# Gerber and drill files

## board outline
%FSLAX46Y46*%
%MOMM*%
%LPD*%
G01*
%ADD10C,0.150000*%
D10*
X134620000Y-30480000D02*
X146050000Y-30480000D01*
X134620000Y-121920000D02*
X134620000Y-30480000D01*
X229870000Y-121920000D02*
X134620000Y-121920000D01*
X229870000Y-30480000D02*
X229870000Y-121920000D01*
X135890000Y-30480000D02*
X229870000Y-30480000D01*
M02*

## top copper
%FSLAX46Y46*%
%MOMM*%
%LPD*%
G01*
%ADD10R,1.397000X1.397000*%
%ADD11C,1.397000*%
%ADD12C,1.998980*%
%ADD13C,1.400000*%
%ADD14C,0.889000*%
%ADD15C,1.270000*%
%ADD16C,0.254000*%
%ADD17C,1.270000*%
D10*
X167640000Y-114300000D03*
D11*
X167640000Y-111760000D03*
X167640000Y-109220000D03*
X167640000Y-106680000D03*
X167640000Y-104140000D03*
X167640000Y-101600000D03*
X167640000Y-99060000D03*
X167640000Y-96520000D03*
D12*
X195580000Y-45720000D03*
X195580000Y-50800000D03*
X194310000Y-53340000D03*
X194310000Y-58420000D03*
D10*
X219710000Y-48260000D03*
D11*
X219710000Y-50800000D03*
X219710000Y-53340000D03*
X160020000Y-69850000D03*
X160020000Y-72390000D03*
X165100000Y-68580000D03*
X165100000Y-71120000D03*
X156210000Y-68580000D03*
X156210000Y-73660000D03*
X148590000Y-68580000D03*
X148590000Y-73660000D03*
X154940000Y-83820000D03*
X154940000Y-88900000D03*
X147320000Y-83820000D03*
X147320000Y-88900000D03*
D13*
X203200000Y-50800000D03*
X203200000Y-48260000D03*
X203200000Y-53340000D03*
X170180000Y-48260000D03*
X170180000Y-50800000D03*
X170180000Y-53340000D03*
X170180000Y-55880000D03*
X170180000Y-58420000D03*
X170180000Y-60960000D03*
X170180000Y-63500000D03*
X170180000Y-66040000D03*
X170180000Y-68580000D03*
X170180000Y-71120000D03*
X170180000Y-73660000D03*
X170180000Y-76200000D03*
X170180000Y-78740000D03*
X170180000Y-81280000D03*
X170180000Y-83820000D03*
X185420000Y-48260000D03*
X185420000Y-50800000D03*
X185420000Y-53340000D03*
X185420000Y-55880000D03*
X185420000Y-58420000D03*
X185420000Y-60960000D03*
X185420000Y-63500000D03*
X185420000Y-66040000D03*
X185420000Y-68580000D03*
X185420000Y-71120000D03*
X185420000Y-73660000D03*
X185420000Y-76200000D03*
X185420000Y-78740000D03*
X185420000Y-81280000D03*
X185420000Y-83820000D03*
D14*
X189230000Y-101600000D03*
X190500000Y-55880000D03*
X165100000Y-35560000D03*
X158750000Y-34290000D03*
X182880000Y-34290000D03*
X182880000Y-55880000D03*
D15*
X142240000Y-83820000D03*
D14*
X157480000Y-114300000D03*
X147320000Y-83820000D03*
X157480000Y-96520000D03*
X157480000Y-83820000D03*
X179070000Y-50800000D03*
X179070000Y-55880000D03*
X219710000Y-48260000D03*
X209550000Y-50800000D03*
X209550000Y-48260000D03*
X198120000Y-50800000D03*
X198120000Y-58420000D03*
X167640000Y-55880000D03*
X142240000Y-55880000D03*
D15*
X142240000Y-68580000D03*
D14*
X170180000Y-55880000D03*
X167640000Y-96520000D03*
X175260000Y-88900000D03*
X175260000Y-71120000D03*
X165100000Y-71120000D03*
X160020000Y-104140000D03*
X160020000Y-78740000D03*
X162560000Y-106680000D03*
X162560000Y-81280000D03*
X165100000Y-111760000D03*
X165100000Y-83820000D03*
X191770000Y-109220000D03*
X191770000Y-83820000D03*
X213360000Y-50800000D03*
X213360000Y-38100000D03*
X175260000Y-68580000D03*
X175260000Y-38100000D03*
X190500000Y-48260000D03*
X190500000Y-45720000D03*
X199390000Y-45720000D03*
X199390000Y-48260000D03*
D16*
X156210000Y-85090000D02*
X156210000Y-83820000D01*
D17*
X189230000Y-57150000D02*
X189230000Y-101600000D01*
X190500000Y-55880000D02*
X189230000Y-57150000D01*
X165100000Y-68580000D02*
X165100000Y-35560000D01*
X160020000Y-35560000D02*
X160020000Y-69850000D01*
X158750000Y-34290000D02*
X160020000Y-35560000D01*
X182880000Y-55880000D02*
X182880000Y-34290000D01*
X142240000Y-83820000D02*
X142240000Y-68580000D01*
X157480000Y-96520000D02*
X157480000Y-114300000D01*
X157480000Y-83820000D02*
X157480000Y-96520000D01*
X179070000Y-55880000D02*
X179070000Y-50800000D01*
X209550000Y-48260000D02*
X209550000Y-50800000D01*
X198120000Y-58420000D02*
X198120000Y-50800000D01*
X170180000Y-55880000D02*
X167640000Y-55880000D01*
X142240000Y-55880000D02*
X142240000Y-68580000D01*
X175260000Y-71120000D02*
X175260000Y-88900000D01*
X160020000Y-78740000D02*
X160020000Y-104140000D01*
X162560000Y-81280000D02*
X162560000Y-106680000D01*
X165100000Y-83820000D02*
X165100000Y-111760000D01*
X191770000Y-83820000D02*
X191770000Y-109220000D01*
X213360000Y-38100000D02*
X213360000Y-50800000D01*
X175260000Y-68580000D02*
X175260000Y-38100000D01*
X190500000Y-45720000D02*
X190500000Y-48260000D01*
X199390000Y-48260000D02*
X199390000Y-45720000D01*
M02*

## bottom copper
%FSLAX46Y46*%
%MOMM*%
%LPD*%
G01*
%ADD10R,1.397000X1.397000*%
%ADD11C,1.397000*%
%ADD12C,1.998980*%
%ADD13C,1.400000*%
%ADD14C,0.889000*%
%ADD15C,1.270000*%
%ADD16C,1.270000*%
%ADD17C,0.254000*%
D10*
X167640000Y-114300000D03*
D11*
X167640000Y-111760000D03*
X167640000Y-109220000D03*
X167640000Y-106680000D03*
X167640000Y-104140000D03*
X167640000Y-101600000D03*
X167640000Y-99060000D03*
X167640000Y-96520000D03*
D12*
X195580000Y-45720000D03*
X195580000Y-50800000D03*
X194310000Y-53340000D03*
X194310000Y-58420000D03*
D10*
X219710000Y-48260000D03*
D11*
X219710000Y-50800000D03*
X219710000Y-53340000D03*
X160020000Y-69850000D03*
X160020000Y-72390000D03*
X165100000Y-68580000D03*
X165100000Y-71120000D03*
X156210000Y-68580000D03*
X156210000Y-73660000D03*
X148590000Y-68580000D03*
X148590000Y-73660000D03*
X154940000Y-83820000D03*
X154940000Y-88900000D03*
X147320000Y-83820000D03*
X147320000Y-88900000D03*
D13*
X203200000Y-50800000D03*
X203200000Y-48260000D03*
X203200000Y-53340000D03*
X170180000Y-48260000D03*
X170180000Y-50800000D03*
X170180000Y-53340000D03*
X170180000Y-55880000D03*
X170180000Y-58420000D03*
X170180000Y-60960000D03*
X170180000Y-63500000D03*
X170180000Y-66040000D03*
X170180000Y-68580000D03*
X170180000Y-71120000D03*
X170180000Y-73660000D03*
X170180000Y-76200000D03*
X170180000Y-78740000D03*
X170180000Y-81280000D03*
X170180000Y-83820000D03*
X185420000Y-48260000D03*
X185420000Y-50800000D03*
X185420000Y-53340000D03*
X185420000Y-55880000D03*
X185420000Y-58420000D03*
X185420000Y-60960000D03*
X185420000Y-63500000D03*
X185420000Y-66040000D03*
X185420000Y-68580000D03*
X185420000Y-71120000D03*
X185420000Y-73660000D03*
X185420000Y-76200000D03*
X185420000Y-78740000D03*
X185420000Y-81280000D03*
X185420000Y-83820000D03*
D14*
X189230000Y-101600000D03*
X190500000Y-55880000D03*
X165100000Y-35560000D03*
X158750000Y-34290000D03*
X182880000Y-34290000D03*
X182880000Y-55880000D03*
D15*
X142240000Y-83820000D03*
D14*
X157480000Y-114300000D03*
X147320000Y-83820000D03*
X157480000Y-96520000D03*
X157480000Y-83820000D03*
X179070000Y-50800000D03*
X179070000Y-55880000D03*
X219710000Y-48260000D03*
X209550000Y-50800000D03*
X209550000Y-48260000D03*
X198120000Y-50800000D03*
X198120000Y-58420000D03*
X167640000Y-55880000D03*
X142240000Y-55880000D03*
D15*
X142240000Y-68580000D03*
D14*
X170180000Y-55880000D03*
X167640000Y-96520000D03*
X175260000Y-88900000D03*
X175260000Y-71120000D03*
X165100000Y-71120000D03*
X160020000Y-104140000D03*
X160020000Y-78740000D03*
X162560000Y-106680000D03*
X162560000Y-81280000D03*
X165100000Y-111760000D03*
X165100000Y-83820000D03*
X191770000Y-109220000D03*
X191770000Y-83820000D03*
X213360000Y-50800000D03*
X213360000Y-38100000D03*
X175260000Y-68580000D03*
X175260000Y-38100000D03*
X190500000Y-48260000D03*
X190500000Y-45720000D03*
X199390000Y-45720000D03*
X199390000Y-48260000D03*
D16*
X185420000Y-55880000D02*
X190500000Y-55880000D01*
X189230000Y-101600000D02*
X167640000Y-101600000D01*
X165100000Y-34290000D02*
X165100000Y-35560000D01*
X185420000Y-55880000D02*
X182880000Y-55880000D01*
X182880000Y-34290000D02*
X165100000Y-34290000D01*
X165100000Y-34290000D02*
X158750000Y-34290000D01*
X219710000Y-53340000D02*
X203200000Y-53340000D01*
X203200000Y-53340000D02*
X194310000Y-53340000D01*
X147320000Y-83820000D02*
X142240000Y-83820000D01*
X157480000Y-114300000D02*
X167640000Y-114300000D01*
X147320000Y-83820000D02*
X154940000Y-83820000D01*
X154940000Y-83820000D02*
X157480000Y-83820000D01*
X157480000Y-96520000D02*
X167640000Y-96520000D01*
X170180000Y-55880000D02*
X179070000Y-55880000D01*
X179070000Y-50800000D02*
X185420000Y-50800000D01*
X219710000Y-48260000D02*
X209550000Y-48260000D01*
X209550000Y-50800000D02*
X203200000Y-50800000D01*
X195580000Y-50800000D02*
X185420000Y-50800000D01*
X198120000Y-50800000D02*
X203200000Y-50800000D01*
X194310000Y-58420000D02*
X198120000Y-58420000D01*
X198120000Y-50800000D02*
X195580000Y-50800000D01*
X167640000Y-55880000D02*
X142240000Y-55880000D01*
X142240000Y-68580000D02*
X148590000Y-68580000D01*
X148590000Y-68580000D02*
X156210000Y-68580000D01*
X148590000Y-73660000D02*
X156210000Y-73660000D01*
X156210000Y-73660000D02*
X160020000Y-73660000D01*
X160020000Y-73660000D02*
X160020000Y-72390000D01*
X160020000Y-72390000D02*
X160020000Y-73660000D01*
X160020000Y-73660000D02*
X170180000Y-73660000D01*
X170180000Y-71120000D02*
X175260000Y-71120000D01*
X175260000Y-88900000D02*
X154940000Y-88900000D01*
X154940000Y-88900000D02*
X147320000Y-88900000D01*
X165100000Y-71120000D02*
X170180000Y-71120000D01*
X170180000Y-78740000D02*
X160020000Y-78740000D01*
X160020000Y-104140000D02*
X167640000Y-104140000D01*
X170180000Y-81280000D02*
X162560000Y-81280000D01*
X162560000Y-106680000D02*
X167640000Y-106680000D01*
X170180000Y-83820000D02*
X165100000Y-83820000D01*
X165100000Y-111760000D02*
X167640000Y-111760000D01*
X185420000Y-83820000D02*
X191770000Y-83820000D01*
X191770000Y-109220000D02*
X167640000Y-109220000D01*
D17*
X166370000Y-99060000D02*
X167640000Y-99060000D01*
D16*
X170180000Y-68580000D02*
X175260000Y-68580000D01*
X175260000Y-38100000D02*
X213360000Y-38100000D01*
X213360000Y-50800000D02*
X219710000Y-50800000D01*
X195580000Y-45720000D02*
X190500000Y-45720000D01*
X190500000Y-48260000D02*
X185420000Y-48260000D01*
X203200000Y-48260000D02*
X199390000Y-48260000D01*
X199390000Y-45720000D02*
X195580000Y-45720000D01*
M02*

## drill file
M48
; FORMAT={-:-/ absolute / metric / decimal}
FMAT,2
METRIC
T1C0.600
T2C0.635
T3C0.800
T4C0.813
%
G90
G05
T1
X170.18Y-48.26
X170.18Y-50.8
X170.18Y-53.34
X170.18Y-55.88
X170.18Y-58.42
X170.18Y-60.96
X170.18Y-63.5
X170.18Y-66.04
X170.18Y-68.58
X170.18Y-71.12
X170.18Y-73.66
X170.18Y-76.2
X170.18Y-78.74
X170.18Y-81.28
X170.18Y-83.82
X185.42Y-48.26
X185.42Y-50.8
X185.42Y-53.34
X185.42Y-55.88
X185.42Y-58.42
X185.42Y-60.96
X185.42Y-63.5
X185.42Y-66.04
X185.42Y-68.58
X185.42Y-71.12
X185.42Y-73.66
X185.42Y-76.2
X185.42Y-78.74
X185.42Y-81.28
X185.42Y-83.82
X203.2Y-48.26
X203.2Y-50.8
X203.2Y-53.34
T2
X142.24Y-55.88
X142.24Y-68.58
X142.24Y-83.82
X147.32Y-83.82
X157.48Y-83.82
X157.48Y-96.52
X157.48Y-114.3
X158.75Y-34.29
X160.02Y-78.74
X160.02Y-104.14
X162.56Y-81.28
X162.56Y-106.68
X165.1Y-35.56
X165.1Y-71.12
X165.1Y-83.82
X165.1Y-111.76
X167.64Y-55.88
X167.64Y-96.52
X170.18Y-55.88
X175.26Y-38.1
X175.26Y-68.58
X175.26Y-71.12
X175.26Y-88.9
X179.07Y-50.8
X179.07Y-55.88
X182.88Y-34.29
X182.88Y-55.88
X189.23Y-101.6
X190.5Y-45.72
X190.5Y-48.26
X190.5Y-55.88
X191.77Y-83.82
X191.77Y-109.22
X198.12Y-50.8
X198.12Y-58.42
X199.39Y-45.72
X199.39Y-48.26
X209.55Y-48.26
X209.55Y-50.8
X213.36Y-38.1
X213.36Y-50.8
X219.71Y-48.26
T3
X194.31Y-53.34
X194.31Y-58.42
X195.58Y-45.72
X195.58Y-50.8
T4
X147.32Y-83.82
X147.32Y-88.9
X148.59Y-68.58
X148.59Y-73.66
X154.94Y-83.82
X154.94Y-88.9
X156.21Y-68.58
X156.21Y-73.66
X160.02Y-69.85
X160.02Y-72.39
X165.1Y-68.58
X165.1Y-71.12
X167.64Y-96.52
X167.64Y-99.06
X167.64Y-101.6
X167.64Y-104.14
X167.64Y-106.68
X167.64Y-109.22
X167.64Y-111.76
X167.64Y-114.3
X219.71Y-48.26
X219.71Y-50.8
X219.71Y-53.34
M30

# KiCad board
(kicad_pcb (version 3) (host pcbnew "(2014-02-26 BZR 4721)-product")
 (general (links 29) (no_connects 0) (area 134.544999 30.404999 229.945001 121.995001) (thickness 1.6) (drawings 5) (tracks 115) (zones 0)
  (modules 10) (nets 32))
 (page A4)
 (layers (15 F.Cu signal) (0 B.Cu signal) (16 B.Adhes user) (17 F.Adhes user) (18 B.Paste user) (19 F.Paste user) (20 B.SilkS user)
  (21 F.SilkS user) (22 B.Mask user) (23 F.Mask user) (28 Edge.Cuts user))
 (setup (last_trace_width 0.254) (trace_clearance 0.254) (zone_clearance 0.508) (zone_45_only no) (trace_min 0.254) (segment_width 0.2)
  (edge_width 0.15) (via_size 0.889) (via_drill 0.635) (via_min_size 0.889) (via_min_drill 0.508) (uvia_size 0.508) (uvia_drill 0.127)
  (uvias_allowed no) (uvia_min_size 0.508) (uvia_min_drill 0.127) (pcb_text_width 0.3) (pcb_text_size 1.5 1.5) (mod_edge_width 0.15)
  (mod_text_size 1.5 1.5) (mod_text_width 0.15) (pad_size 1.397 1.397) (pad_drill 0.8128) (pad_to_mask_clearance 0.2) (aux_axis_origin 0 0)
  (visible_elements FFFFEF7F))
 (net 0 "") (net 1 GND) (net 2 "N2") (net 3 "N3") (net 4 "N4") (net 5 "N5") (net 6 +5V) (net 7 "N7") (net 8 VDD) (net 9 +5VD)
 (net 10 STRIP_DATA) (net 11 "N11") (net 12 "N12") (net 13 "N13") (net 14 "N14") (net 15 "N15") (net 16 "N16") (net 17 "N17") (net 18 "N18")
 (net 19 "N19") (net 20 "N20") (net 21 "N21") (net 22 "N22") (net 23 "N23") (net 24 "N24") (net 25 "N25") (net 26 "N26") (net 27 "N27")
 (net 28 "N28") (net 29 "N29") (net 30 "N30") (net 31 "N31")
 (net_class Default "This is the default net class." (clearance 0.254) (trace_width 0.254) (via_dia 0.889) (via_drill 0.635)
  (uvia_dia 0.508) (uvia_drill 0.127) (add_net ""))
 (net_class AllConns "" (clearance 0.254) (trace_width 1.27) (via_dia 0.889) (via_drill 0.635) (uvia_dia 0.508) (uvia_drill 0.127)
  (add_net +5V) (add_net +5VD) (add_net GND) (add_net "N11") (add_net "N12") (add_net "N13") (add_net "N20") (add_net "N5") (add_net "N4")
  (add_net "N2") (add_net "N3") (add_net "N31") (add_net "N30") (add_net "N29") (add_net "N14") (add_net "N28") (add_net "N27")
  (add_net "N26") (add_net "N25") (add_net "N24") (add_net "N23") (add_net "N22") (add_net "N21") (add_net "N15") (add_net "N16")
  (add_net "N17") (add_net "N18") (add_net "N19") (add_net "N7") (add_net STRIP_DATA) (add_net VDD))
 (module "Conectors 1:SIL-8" (layer F.Cu) (at 167.64 105.41 90)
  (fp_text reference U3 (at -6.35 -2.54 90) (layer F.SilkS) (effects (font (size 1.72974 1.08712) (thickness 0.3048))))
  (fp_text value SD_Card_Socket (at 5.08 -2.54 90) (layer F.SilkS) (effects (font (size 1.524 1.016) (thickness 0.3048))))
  (pad 8 thru_hole rect (at -8.89 0 90) (size 1.397 1.397) (drill 0.8128) (layers *.Cu *.Mask F.SilkS) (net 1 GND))
  (pad 7 thru_hole circle (at -6.35 0 90) (size 1.397 1.397) (drill 0.8128) (layers *.Cu *.Mask F.SilkS) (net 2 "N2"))
  (pad 6 thru_hole circle (at -3.81 0 90) (size 1.397 1.397) (drill 0.8128) (layers *.Cu *.Mask F.SilkS) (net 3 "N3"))
  (pad 5 thru_hole circle (at -1.27 0 90) (size 1.397 1.397) (drill 0.8128) (layers *.Cu *.Mask F.SilkS) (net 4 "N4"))
  (pad 4 thru_hole circle (at 1.27 0 90) (size 1.397 1.397) (drill 0.8128) (layers *.Cu *.Mask F.SilkS) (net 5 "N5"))
  (pad 3 thru_hole circle (at 3.81 0 90) (size 1.397 1.397) (drill 0.8128) (layers *.Cu *.Mask F.SilkS) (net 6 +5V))
  (pad 2 thru_hole circle (at 6.35 0 90) (size 1.397 1.397) (drill 0.8128) (layers *.Cu *.Mask F.SilkS) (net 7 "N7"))
  (pad 1 thru_hole circle (at 8.89 0 90) (size 1.397 1.397) (drill 0.8128) (layers *.Cu *.Mask F.SilkS) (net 1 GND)))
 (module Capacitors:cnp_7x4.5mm (layer F.Cu) (at 195.58 48.26 270)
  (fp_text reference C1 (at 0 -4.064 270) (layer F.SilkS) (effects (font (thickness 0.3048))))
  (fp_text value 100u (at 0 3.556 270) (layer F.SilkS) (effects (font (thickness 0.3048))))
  (pad 1 thru_hole circle (at -2.54 0 270) (size 1.99898 1.99898) (drill 0.8001) (layers *.Cu *.Mask F.SilkS) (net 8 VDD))
  (pad 2 thru_hole circle (at 2.54 0 270) (size 1.99898 1.99898) (drill 0.8001) (layers *.Cu *.Mask F.SilkS) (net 1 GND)))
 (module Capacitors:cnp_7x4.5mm (layer F.Cu) (at 194.31 55.88 270)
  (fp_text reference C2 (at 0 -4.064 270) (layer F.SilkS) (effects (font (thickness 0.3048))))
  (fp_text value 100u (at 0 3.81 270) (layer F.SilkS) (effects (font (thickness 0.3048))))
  (pad 1 thru_hole circle (at -2.54 0 270) (size 1.99898 1.99898) (drill 0.8001) (layers *.Cu *.Mask F.SilkS) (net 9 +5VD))
  (pad 2 thru_hole circle (at 2.54 0 270) (size 1.99898 1.99898) (drill 0.8001) (layers *.Cu *.Mask F.SilkS) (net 1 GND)))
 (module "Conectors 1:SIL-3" (layer F.Cu) (at 219.71 50.8 270)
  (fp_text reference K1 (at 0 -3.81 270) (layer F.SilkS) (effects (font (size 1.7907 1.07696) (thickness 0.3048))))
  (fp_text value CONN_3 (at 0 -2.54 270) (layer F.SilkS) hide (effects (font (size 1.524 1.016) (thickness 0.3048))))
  (pad 1 thru_hole rect (at -2.54 0 270) (size 1.397 1.397) (drill 0.8128) (layers *.Cu *.Mask F.SilkS) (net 1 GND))
  (pad 2 thru_hole circle (at 0 0 270) (size 1.397 1.397) (drill 0.8128) (layers *.Cu *.Mask F.SilkS) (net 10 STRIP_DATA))
  (pad 3 thru_hole circle (at 2.54 0 270) (size 1.397 1.397) (drill 0.8128) (layers *.Cu *.Mask F.SilkS) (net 9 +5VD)))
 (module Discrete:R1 (layer F.Cu) (at 160.02 71.12 270) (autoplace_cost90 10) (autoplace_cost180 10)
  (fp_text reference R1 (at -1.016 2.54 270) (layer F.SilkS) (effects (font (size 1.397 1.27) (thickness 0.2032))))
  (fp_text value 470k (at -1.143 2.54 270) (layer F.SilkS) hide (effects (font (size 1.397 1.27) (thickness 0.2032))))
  (pad 1 thru_hole circle (at -1.27 0 270) (size 1.397 1.397) (drill 0.8128) (layers *.Cu *.Mask F.SilkS) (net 6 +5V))
  (pad 2 thru_hole circle (at 1.27 0 270) (size 1.397 1.397) (drill 0.8128) (layers *.Cu *.Mask F.SilkS) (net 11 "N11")))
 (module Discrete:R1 (layer F.Cu) (at 165.1 69.85 270) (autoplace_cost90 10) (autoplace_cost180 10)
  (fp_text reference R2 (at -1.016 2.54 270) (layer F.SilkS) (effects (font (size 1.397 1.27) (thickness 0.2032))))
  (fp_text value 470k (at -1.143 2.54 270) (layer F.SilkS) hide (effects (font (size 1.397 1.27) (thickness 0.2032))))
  (pad 1 thru_hole circle (at -1.27 0 270) (size 1.397 1.397) (drill 0.8128) (layers *.Cu *.Mask F.SilkS) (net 6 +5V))
  (pad 2 thru_hole circle (at 1.27 0 270) (size 1.397 1.397) (drill 0.8128) (layers *.Cu *.Mask F.SilkS) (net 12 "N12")))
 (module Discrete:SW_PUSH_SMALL (layer F.Cu) (at 152.4 71.12)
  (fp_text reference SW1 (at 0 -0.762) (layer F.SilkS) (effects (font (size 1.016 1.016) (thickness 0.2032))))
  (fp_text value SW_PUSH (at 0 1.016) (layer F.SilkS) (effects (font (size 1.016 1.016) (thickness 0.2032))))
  (pad 1 thru_hole circle (at 3.81 -2.54) (size 1.397 1.397) (drill 0.8128) (layers *.Cu *.Mask F.SilkS) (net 1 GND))
  (pad 2 thru_hole circle (at 3.81 2.54) (size 1.397 1.397) (drill 0.8128) (layers *.Cu *.Mask F.SilkS) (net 11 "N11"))
  (pad 1 thru_hole circle (at -3.81 -2.54) (size 1.397 1.397) (drill 0.8128) (layers *.Cu *.Mask F.SilkS) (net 1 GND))
  (pad 2 thru_hole circle (at -3.81 2.54) (size 1.397 1.397) (drill 0.8128) (layers *.Cu *.Mask F.SilkS) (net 11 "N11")))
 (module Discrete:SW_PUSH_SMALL (layer F.Cu) (at 151.13 86.36)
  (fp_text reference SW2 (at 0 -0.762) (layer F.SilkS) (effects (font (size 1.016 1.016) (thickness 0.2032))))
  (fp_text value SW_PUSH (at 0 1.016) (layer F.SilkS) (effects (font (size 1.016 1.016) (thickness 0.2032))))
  (pad 1 thru_hole circle (at 3.81 -2.54) (size 1.397 1.397) (drill 0.8128) (layers *.Cu *.Mask F.SilkS) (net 1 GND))
  (pad 2 thru_hole circle (at 3.81 2.54) (size 1.397 1.397) (drill 0.8128) (layers *.Cu *.Mask F.SilkS) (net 12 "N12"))
  (pad 1 thru_hole circle (at -3.81 -2.54) (size 1.397 1.397) (drill 0.8128) (layers *.Cu *.Mask F.SilkS) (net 1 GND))
  (pad 2 thru_hole circle (at -3.81 2.54) (size 1.397 1.397) (drill 0.8128) (layers *.Cu *.Mask F.SilkS) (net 12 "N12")))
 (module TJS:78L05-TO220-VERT (layer F.Cu) (at 208.28 50.8 270)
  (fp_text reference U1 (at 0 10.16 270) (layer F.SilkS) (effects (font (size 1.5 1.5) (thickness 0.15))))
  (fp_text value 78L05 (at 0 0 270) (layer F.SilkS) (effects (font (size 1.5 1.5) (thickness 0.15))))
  (pad 1 thru_hole circle (at 0 5.08 270) (size 1.4 1.4) (drill 0.6) (layers *.Cu *.Mask F.SilkS) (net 1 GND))
  (pad 2 thru_hole circle (at -2.54 5.08 270) (size 1.4 1.4) (drill 0.6) (layers *.Cu *.Mask F.SilkS) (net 8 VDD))
  (pad 3 thru_hole circle (at 2.54 5.08 270) (size 1.4 1.4) (drill 0.6) (layers *.Cu *.Mask F.SilkS) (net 9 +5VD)))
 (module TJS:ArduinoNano (layer F.Cu) (at 177.8 45.72)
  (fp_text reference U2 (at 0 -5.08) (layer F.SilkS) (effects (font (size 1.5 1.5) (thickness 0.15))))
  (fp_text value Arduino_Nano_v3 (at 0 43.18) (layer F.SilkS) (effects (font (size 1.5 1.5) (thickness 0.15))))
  (pad 1 thru_hole circle (at -7.62 2.54) (size 1.4 1.4) (drill 0.6) (layers *.Cu *.Mask F.SilkS) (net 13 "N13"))
  (pad 2 thru_hole circle (at -7.62 5.08) (size 1.4 1.4) (drill 0.6) (layers *.Cu *.Mask F.SilkS) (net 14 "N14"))
  (pad 3 thru_hole circle (at -7.62 7.62) (size 1.4 1.4) (drill 0.6) (layers *.Cu *.Mask F.SilkS) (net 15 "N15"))
  (pad 4 thru_hole circle (at -7.62 10.16) (size 1.4 1.4) (drill 0.6) (layers *.Cu *.Mask F.SilkS) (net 1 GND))
  (pad 5 thru_hole circle (at -7.62 12.7) (size 1.4 1.4) (drill 0.6) (layers *.Cu *.Mask F.SilkS) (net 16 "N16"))
  (pad 6 thru_hole circle (at -7.62 15.24) (size 1.4 1.4) (drill 0.6) (layers *.Cu *.Mask F.SilkS) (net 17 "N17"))
  (pad 7 thru_hole circle (at -7.62 17.78) (size 1.4 1.4) (drill 0.6) (layers *.Cu *.Mask F.SilkS) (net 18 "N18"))
  (pad 8 thru_hole circle (at -7.62 20.32) (size 1.4 1.4) (drill 0.6) (layers *.Cu *.Mask F.SilkS) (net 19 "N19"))
  (pad 9 thru_hole circle (at -7.62 22.86) (size 1.4 1.4) (drill 0.6) (layers *.Cu *.Mask F.SilkS) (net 10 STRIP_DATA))
  (pad 10 thru_hole circle (at -7.62 25.4) (size 1.4 1.4) (drill 0.6) (layers *.Cu *.Mask F.SilkS) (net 12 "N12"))
  (pad 11 thru_hole circle (at -7.62 27.94) (size 1.4 1.4) (drill 0.6) (layers *.Cu *.Mask F.SilkS) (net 11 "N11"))
  (pad 12 thru_hole circle (at -7.62 30.48) (size 1.4 1.4) (drill 0.6) (layers *.Cu *.Mask F.SilkS) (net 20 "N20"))
  (pad 13 thru_hole circle (at -7.62 33.02) (size 1.4 1.4) (drill 0.6) (layers *.Cu *.Mask F.SilkS) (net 5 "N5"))
  (pad 14 thru_hole circle (at -7.62 35.56) (size 1.4 1.4) (drill 0.6) (layers *.Cu *.Mask F.SilkS) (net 4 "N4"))
  (pad 15 thru_hole circle (at -7.62 38.1) (size 1.4 1.4) (drill 0.6) (layers *.Cu *.Mask F.SilkS) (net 2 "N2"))
  (pad 30 thru_hole circle (at 7.62 2.54) (size 1.4 1.4) (drill 0.6) (layers *.Cu *.Mask F.SilkS) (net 8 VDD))
  (pad 29 thru_hole circle (at 7.62 5.08) (size 1.4 1.4) (drill 0.6) (layers *.Cu *.Mask F.SilkS) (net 1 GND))
  (pad 28 thru_hole circle (at 7.62 7.62) (size 1.4 1.4) (drill 0.6) (layers *.Cu *.Mask F.SilkS) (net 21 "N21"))
  (pad 27 thru_hole circle (at 7.62 10.16) (size 1.4 1.4) (drill 0.6) (layers *.Cu *.Mask F.SilkS) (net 6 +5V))
  (pad 26 thru_hole circle (at 7.62 12.7) (size 1.4 1.4) (drill 0.6) (layers *.Cu *.Mask F.SilkS) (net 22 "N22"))
  (pad 25 thru_hole circle (at 7.62 15.24) (size 1.4 1.4) (drill 0.6) (layers *.Cu *.Mask F.SilkS) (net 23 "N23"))
  (pad 24 thru_hole circle (at 7.62 17.78) (size 1.4 1.4) (drill 0.6) (layers *.Cu *.Mask F.SilkS) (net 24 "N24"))
  (pad 23 thru_hole circle (at 7.62 20.32) (size 1.4 1.4) (drill 0.6) (layers *.Cu *.Mask F.SilkS) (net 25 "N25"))
  (pad 22 thru_hole circle (at 7.62 22.86) (size 1.4 1.4) (drill 0.6) (layers *.Cu *.Mask F.SilkS) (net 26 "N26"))
  (pad 21 thru_hole circle (at 7.62 25.4) (size 1.4 1.4) (drill 0.6) (layers *.Cu *.Mask F.SilkS) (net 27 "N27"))
  (pad 20 thru_hole circle (at 7.62 27.94) (size 1.4 1.4) (drill 0.6) (layers *.Cu *.Mask F.SilkS) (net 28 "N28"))
  (pad 19 thru_hole circle (at 7.62 30.48) (size 1.4 1.4) (drill 0.6) (layers *.Cu *.Mask F.SilkS) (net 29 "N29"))
  (pad 18 thru_hole circle (at 7.62 33.02) (size 1.4 1.4) (drill 0.6) (layers *.Cu *.Mask F.SilkS) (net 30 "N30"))
  (pad 17 thru_hole circle (at 7.62 35.56) (size 1.4 1.4) (drill 0.6) (layers *.Cu *.Mask F.SilkS) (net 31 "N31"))
  (pad 16 thru_hole circle (at 7.62 38.1) (size 1.4 1.4) (drill 0.6) (layers *.Cu *.Mask F.SilkS) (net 3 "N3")))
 (gr_line (start 134.62 30.48) (end 146.05 30.48) (angle 90) (layer Edge.Cuts) (width 0.15))
 (gr_line (start 134.62 121.92) (end 134.62 30.48) (angle 90) (layer Edge.Cuts) (width 0.15))
 (gr_line (start 229.87 121.92) (end 134.62 121.92) (angle 90) (layer Edge.Cuts) (width 0.15))
 (gr_line (start 229.87 30.48) (end 229.87 121.92) (angle 90) (layer Edge.Cuts) (width 0.15))
 (gr_line (start 135.89 30.48) (end 229.87 30.48) (angle 90) (layer Edge.Cuts) (width 0.15))
 (segment (start 156.21 85.09) (end 156.21 83.82) (width 0.254) (layer F.Cu) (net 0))
 (segment (start 185.42 55.88) (end 190.5 55.88) (width 1.27) (layer B.Cu) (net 6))
 (segment (start 189.23 101.6) (end 167.64 101.6) (width 1.27) (layer B.Cu) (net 6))
 (via (at 189.23 101.6) (size 0.889) (layers F.Cu B.Cu) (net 6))
 (segment (start 189.23 57.15) (end 189.23 101.6) (width 1.27) (layer F.Cu) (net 6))
 (segment (start 190.5 55.88) (end 189.23 57.15) (width 1.27) (layer F.Cu) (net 6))
 (via (at 190.5 55.88) (size 0.889) (layers F.Cu B.Cu) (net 6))
 (segment (start 165.1 34.29) (end 165.1 35.56) (width 1.27) (layer B.Cu) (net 6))
 (via (at 165.1 35.56) (size 0.889) (layers F.Cu B.Cu) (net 6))
 (segment (start 165.1 68.58) (end 165.1 35.56) (width 1.27) (layer F.Cu) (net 6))
 (segment (start 185.42 55.88) (end 182.88 55.88) (width 1.27) (layer B.Cu) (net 6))
 (segment (start 160.02 35.56) (end 160.02 69.85) (width 1.27) (layer F.Cu) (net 6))
 (segment (start 158.75 34.29) (end 160.02 35.56) (width 1.27) (layer F.Cu) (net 6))
 (via (at 158.75 34.29) (size 0.889) (layers F.Cu B.Cu) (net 6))
 (segment (start 182.88 34.29) (end 165.1 34.29) (width 1.27) (layer B.Cu) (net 6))
 (segment (start 165.1 34.29) (end 158.75 34.29) (width 1.27) (layer B.Cu) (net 6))
 (via (at 182.88 34.29) (size 0.889) (layers F.Cu B.Cu) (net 6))
 (segment (start 182.88 55.88) (end 182.88 34.29) (width 1.27) (layer F.Cu) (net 6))
 (via (at 182.88 55.88) (size 0.889) (layers F.Cu B.Cu) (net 6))
 (segment (start 219.71 53.34) (end 203.2 53.34) (width 1.27) (layer B.Cu) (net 9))
 (segment (start 203.2 53.34) (end 194.31 53.34) (width 1.27) (layer B.Cu) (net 9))
 (segment (start 147.32 83.82) (end 142.24 83.82) (width 1.27) (layer B.Cu) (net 1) (status 400000))
 (via (at 142.24 83.82) (size 1.27) (layers F.Cu B.Cu) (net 1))
 (segment (start 142.24 83.82) (end 142.24 68.58) (width 1.27) (layer F.Cu) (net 1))
 (segment (start 157.48 96.52) (end 157.48 114.3) (width 1.27) (layer F.Cu) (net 1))
 (segment (start 157.48 114.3) (end 167.64 114.3) (width 1.27) (layer B.Cu) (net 1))
 (via (at 157.48 114.3) (size 0.889) (layers F.Cu B.Cu) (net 1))
 (via (at 147.32 83.82) (size 0.889) (layers F.Cu B.Cu) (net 1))
 (segment (start 147.32 83.82) (end 154.94 83.82) (width 1.27) (layer B.Cu) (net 1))
 (segment (start 154.94 83.82) (end 157.48 83.82) (width 1.27) (layer B.Cu) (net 1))
 (segment (start 157.48 96.52) (end 167.64 96.52) (width 1.27) (layer B.Cu) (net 1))
 (via (at 157.48 96.52) (size 0.889) (layers F.Cu B.Cu) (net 1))
 (segment (start 157.48 83.82) (end 157.48 96.52) (width 1.27) (layer F.Cu) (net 1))
 (via (at 157.48 83.82) (size 0.889) (layers F.Cu B.Cu) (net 1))
 (segment (start 170.18 55.88) (end 179.07 55.88) (width 1.27) (layer B.Cu) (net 1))
 (segment (start 179.07 50.8) (end 185.42 50.8) (width 1.27) (layer B.Cu) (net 1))
 (via (at 179.07 50.8) (size 0.889) (layers F.Cu B.Cu) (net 1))
 (segment (start 179.07 55.88) (end 179.07 50.8) (width 1.27) (layer F.Cu) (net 1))
 (via (at 179.07 55.88) (size 0.889) (layers F.Cu B.Cu) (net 1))
 (via (at 219.71 48.26) (size 0.889) (layers F.Cu B.Cu) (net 1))
 (segment (start 219.71 48.26) (end 209.55 48.26) (width 1.27) (layer B.Cu) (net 1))
 (segment (start 209.55 50.8) (end 203.2 50.8) (width 1.27) (layer B.Cu) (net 1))
 (via (at 209.55 50.8) (size 0.889) (layers F.Cu B.Cu) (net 1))
 (segment (start 209.55 48.26) (end 209.55 50.8) (width 1.27) (layer F.Cu) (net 1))
 (via (at 209.55 48.26) (size 0.889) (layers F.Cu B.Cu) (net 1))
 (segment (start 195.58 50.8) (end 185.42 50.8) (width 1.27) (layer B.Cu) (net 1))
 (segment (start 198.12 50.8) (end 203.2 50.8) (width 1.27) (layer B.Cu) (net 1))
 (segment (start 194.31 58.42) (end 198.12 58.42) (width 1.27) (layer B.Cu) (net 1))
 (segment (start 198.12 50.8) (end 195.58 50.8) (width 1.27) (layer B.Cu) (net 1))
 (via (at 198.12 50.8) (size 0.889) (layers F.Cu B.Cu) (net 1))
 (segment (start 198.12 58.42) (end 198.12 50.8) (width 1.27) (layer F.Cu) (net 1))
 (via (at 198.12 58.42) (size 0.889) (layers F.Cu B.Cu) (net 1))
 (segment (start 170.18 55.88) (end 167.64 55.88) (width 1.27) (layer F.Cu) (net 1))
 (via (at 167.64 55.88) (size 0.889) (layers F.Cu B.Cu) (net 1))
 (segment (start 167.64 55.88) (end 142.24 55.88) (width 1.27) (layer B.Cu) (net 1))
 (via (at 142.24 55.88) (size 0.889) (layers F.Cu B.Cu) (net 1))
 (segment (start 142.24 55.88) (end 142.24 68.58) (width 1.27) (layer F.Cu) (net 1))
 (segment (start 142.24 68.58) (end 148.59 68.58) (width 1.27) (layer B.Cu) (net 1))
 (via (at 142.24 68.58) (size 1.27) (layers F.Cu B.Cu) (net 1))
 (segment (start 148.59 68.58) (end 156.21 68.58) (width 1.27) (layer B.Cu) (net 1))
 (via (at 170.18 55.88) (size 0.889) (layers F.Cu B.Cu) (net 1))
 (via (at 167.64 96.52) (size 0.889) (layers F.Cu B.Cu) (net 1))
 (segment (start 148.59 73.66) (end 156.21 73.66) (width 1.27) (layer B.Cu) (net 11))
 (segment (start 156.21 73.66) (end 160.02 73.66) (width 1.27) (layer B.Cu) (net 11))
 (segment (start 160.02 73.66) (end 160.02 72.39) (width 1.27) (layer B.Cu) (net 11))
 (segment (start 160.02 72.39) (end 160.02 73.66) (width 1.27) (layer B.Cu) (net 11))
 (segment (start 160.02 73.66) (end 170.18 73.66) (width 1.27) (layer B.Cu) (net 11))
 (segment (start 170.18 71.12) (end 175.26 71.12) (width 1.27) (layer B.Cu) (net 12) (status 400000))
 (segment (start 175.26 88.9) (end 154.94 88.9) (width 1.27) (layer B.Cu) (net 12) (status 800000))
 (via (at 175.26 88.9) (size 0.889) (layers F.Cu B.Cu) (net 12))
 (segment (start 175.26 71.12) (end 175.26 88.9) (width 1.27) (layer F.Cu) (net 12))
 (via (at 175.26 71.12) (size 0.889) (layers F.Cu B.Cu) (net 12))
 (segment (start 154.94 88.9) (end 147.32 88.9) (width 1.27) (layer B.Cu) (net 12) (status C00000))
 (via (at 165.1 71.12) (size 0.889) (layers F.Cu B.Cu) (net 12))
 (segment (start 165.1 71.12) (end 170.18 71.12) (width 1.27) (layer B.Cu) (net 12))
 (segment (start 170.18 78.74) (end 160.02 78.74) (width 1.27) (layer B.Cu) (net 5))
 (segment (start 160.02 104.14) (end 167.64 104.14) (width 1.27) (layer B.Cu) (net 5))
 (via (at 160.02 104.14) (size 0.889) (layers F.Cu B.Cu) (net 5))
 (segment (start 160.02 78.74) (end 160.02 104.14) (width 1.27) (layer F.Cu) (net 5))
 (via (at 160.02 78.74) (size 0.889) (layers F.Cu B.Cu) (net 5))
 (segment (start 170.18 81.28) (end 162.56 81.28) (width 1.27) (layer B.Cu) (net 4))
 (segment (start 162.56 106.68) (end 167.64 106.68) (width 1.27) (layer B.Cu) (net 4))
 (via (at 162.56 106.68) (size 0.889) (layers F.Cu B.Cu) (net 4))
 (segment (start 162.56 81.28) (end 162.56 106.68) (width 1.27) (layer F.Cu) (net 4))
 (via (at 162.56 81.28) (size 0.889) (layers F.Cu B.Cu) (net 4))
 (segment (start 170.18 83.82) (end 165.1 83.82) (width 1.27) (layer B.Cu) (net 2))
 (segment (start 165.1 111.76) (end 167.64 111.76) (width 1.27) (layer B.Cu) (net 2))
 (via (at 165.1 111.76) (size 0.889) (layers F.Cu B.Cu) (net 2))
 (segment (start 165.1 83.82) (end 165.1 111.76) (width 1.27) (layer F.Cu) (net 2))
 (via (at 165.1 83.82) (size 0.889) (layers F.Cu B.Cu) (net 2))
 (segment (start 185.42 83.82) (end 191.77 83.82) (width 1.27) (layer B.Cu) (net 3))
 (segment (start 191.77 109.22) (end 167.64 109.22) (width 1.27) (layer B.Cu) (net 3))
 (via (at 191.77 109.22) (size 0.889) (layers F.Cu B.Cu) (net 3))
 (segment (start 191.77 83.82) (end 191.77 109.22) (width 1.27) (layer F.Cu) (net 3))
 (via (at 191.77 83.82) (size 0.889) (layers F.Cu B.Cu) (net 3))
 (segment (start 166.37 99.06) (end 167.64 99.06) (width 0.254) (layer B.Cu) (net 7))
 (via (at 213.36 50.8) (size 0.889) (layers F.Cu B.Cu) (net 10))
 (via (at 213.36 38.1) (size 0.889) (layers F.Cu B.Cu) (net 10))
 (segment (start 213.36 38.1) (end 213.36 50.8) (width 1.27) (layer F.Cu) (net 10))
 (via (at 175.26 68.58) (size 0.889) (layers F.Cu B.Cu) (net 10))
 (segment (start 175.26 68.58) (end 175.26 38.1) (width 1.27) (layer F.Cu) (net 10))
 (via (at 175.26 38.1) (size 0.889) (layers F.Cu B.Cu) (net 10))
 (segment (start 170.18 68.58) (end 175.26 68.58) (width 1.27) (layer B.Cu) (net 10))
 (segment (start 175.26 38.1) (end 213.36 38.1) (width 1.27) (layer B.Cu) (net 10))
 (segment (start 213.36 50.8) (end 219.71 50.8) (width 1.27) (layer B.Cu) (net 10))
 (segment (start 195.58 45.72) (end 190.5 45.72) (width 1.27) (layer B.Cu) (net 8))
 (segment (start 190.5 48.26) (end 185.42 48.26) (width 1.27) (layer B.Cu) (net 8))
 (via (at 190.5 48.26) (size 0.889) (layers F.Cu B.Cu) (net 8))
 (segment (start 190.5 45.72) (end 190.5 48.26) (width 1.27) (layer F.Cu) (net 8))
 (via (at 190.5 45.72) (size 0.889) (layers F.Cu B.Cu) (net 8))
 (segment (start 203.2 48.26) (end 199.39 48.26) (width 1.27) (layer B.Cu) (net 8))
 (segment (start 199.39 45.72) (end 195.58 45.72) (width 1.27) (layer B.Cu) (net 8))
 (via (at 199.39 45.72) (size 0.889) (layers F.Cu B.Cu) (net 8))
 (segment (start 199.39 48.26) (end 199.39 45.72) (width 1.27) (layer F.Cu) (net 8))
 (via (at 199.39 48.26) (size 0.889) (layers F.Cu B.Cu) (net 8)))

